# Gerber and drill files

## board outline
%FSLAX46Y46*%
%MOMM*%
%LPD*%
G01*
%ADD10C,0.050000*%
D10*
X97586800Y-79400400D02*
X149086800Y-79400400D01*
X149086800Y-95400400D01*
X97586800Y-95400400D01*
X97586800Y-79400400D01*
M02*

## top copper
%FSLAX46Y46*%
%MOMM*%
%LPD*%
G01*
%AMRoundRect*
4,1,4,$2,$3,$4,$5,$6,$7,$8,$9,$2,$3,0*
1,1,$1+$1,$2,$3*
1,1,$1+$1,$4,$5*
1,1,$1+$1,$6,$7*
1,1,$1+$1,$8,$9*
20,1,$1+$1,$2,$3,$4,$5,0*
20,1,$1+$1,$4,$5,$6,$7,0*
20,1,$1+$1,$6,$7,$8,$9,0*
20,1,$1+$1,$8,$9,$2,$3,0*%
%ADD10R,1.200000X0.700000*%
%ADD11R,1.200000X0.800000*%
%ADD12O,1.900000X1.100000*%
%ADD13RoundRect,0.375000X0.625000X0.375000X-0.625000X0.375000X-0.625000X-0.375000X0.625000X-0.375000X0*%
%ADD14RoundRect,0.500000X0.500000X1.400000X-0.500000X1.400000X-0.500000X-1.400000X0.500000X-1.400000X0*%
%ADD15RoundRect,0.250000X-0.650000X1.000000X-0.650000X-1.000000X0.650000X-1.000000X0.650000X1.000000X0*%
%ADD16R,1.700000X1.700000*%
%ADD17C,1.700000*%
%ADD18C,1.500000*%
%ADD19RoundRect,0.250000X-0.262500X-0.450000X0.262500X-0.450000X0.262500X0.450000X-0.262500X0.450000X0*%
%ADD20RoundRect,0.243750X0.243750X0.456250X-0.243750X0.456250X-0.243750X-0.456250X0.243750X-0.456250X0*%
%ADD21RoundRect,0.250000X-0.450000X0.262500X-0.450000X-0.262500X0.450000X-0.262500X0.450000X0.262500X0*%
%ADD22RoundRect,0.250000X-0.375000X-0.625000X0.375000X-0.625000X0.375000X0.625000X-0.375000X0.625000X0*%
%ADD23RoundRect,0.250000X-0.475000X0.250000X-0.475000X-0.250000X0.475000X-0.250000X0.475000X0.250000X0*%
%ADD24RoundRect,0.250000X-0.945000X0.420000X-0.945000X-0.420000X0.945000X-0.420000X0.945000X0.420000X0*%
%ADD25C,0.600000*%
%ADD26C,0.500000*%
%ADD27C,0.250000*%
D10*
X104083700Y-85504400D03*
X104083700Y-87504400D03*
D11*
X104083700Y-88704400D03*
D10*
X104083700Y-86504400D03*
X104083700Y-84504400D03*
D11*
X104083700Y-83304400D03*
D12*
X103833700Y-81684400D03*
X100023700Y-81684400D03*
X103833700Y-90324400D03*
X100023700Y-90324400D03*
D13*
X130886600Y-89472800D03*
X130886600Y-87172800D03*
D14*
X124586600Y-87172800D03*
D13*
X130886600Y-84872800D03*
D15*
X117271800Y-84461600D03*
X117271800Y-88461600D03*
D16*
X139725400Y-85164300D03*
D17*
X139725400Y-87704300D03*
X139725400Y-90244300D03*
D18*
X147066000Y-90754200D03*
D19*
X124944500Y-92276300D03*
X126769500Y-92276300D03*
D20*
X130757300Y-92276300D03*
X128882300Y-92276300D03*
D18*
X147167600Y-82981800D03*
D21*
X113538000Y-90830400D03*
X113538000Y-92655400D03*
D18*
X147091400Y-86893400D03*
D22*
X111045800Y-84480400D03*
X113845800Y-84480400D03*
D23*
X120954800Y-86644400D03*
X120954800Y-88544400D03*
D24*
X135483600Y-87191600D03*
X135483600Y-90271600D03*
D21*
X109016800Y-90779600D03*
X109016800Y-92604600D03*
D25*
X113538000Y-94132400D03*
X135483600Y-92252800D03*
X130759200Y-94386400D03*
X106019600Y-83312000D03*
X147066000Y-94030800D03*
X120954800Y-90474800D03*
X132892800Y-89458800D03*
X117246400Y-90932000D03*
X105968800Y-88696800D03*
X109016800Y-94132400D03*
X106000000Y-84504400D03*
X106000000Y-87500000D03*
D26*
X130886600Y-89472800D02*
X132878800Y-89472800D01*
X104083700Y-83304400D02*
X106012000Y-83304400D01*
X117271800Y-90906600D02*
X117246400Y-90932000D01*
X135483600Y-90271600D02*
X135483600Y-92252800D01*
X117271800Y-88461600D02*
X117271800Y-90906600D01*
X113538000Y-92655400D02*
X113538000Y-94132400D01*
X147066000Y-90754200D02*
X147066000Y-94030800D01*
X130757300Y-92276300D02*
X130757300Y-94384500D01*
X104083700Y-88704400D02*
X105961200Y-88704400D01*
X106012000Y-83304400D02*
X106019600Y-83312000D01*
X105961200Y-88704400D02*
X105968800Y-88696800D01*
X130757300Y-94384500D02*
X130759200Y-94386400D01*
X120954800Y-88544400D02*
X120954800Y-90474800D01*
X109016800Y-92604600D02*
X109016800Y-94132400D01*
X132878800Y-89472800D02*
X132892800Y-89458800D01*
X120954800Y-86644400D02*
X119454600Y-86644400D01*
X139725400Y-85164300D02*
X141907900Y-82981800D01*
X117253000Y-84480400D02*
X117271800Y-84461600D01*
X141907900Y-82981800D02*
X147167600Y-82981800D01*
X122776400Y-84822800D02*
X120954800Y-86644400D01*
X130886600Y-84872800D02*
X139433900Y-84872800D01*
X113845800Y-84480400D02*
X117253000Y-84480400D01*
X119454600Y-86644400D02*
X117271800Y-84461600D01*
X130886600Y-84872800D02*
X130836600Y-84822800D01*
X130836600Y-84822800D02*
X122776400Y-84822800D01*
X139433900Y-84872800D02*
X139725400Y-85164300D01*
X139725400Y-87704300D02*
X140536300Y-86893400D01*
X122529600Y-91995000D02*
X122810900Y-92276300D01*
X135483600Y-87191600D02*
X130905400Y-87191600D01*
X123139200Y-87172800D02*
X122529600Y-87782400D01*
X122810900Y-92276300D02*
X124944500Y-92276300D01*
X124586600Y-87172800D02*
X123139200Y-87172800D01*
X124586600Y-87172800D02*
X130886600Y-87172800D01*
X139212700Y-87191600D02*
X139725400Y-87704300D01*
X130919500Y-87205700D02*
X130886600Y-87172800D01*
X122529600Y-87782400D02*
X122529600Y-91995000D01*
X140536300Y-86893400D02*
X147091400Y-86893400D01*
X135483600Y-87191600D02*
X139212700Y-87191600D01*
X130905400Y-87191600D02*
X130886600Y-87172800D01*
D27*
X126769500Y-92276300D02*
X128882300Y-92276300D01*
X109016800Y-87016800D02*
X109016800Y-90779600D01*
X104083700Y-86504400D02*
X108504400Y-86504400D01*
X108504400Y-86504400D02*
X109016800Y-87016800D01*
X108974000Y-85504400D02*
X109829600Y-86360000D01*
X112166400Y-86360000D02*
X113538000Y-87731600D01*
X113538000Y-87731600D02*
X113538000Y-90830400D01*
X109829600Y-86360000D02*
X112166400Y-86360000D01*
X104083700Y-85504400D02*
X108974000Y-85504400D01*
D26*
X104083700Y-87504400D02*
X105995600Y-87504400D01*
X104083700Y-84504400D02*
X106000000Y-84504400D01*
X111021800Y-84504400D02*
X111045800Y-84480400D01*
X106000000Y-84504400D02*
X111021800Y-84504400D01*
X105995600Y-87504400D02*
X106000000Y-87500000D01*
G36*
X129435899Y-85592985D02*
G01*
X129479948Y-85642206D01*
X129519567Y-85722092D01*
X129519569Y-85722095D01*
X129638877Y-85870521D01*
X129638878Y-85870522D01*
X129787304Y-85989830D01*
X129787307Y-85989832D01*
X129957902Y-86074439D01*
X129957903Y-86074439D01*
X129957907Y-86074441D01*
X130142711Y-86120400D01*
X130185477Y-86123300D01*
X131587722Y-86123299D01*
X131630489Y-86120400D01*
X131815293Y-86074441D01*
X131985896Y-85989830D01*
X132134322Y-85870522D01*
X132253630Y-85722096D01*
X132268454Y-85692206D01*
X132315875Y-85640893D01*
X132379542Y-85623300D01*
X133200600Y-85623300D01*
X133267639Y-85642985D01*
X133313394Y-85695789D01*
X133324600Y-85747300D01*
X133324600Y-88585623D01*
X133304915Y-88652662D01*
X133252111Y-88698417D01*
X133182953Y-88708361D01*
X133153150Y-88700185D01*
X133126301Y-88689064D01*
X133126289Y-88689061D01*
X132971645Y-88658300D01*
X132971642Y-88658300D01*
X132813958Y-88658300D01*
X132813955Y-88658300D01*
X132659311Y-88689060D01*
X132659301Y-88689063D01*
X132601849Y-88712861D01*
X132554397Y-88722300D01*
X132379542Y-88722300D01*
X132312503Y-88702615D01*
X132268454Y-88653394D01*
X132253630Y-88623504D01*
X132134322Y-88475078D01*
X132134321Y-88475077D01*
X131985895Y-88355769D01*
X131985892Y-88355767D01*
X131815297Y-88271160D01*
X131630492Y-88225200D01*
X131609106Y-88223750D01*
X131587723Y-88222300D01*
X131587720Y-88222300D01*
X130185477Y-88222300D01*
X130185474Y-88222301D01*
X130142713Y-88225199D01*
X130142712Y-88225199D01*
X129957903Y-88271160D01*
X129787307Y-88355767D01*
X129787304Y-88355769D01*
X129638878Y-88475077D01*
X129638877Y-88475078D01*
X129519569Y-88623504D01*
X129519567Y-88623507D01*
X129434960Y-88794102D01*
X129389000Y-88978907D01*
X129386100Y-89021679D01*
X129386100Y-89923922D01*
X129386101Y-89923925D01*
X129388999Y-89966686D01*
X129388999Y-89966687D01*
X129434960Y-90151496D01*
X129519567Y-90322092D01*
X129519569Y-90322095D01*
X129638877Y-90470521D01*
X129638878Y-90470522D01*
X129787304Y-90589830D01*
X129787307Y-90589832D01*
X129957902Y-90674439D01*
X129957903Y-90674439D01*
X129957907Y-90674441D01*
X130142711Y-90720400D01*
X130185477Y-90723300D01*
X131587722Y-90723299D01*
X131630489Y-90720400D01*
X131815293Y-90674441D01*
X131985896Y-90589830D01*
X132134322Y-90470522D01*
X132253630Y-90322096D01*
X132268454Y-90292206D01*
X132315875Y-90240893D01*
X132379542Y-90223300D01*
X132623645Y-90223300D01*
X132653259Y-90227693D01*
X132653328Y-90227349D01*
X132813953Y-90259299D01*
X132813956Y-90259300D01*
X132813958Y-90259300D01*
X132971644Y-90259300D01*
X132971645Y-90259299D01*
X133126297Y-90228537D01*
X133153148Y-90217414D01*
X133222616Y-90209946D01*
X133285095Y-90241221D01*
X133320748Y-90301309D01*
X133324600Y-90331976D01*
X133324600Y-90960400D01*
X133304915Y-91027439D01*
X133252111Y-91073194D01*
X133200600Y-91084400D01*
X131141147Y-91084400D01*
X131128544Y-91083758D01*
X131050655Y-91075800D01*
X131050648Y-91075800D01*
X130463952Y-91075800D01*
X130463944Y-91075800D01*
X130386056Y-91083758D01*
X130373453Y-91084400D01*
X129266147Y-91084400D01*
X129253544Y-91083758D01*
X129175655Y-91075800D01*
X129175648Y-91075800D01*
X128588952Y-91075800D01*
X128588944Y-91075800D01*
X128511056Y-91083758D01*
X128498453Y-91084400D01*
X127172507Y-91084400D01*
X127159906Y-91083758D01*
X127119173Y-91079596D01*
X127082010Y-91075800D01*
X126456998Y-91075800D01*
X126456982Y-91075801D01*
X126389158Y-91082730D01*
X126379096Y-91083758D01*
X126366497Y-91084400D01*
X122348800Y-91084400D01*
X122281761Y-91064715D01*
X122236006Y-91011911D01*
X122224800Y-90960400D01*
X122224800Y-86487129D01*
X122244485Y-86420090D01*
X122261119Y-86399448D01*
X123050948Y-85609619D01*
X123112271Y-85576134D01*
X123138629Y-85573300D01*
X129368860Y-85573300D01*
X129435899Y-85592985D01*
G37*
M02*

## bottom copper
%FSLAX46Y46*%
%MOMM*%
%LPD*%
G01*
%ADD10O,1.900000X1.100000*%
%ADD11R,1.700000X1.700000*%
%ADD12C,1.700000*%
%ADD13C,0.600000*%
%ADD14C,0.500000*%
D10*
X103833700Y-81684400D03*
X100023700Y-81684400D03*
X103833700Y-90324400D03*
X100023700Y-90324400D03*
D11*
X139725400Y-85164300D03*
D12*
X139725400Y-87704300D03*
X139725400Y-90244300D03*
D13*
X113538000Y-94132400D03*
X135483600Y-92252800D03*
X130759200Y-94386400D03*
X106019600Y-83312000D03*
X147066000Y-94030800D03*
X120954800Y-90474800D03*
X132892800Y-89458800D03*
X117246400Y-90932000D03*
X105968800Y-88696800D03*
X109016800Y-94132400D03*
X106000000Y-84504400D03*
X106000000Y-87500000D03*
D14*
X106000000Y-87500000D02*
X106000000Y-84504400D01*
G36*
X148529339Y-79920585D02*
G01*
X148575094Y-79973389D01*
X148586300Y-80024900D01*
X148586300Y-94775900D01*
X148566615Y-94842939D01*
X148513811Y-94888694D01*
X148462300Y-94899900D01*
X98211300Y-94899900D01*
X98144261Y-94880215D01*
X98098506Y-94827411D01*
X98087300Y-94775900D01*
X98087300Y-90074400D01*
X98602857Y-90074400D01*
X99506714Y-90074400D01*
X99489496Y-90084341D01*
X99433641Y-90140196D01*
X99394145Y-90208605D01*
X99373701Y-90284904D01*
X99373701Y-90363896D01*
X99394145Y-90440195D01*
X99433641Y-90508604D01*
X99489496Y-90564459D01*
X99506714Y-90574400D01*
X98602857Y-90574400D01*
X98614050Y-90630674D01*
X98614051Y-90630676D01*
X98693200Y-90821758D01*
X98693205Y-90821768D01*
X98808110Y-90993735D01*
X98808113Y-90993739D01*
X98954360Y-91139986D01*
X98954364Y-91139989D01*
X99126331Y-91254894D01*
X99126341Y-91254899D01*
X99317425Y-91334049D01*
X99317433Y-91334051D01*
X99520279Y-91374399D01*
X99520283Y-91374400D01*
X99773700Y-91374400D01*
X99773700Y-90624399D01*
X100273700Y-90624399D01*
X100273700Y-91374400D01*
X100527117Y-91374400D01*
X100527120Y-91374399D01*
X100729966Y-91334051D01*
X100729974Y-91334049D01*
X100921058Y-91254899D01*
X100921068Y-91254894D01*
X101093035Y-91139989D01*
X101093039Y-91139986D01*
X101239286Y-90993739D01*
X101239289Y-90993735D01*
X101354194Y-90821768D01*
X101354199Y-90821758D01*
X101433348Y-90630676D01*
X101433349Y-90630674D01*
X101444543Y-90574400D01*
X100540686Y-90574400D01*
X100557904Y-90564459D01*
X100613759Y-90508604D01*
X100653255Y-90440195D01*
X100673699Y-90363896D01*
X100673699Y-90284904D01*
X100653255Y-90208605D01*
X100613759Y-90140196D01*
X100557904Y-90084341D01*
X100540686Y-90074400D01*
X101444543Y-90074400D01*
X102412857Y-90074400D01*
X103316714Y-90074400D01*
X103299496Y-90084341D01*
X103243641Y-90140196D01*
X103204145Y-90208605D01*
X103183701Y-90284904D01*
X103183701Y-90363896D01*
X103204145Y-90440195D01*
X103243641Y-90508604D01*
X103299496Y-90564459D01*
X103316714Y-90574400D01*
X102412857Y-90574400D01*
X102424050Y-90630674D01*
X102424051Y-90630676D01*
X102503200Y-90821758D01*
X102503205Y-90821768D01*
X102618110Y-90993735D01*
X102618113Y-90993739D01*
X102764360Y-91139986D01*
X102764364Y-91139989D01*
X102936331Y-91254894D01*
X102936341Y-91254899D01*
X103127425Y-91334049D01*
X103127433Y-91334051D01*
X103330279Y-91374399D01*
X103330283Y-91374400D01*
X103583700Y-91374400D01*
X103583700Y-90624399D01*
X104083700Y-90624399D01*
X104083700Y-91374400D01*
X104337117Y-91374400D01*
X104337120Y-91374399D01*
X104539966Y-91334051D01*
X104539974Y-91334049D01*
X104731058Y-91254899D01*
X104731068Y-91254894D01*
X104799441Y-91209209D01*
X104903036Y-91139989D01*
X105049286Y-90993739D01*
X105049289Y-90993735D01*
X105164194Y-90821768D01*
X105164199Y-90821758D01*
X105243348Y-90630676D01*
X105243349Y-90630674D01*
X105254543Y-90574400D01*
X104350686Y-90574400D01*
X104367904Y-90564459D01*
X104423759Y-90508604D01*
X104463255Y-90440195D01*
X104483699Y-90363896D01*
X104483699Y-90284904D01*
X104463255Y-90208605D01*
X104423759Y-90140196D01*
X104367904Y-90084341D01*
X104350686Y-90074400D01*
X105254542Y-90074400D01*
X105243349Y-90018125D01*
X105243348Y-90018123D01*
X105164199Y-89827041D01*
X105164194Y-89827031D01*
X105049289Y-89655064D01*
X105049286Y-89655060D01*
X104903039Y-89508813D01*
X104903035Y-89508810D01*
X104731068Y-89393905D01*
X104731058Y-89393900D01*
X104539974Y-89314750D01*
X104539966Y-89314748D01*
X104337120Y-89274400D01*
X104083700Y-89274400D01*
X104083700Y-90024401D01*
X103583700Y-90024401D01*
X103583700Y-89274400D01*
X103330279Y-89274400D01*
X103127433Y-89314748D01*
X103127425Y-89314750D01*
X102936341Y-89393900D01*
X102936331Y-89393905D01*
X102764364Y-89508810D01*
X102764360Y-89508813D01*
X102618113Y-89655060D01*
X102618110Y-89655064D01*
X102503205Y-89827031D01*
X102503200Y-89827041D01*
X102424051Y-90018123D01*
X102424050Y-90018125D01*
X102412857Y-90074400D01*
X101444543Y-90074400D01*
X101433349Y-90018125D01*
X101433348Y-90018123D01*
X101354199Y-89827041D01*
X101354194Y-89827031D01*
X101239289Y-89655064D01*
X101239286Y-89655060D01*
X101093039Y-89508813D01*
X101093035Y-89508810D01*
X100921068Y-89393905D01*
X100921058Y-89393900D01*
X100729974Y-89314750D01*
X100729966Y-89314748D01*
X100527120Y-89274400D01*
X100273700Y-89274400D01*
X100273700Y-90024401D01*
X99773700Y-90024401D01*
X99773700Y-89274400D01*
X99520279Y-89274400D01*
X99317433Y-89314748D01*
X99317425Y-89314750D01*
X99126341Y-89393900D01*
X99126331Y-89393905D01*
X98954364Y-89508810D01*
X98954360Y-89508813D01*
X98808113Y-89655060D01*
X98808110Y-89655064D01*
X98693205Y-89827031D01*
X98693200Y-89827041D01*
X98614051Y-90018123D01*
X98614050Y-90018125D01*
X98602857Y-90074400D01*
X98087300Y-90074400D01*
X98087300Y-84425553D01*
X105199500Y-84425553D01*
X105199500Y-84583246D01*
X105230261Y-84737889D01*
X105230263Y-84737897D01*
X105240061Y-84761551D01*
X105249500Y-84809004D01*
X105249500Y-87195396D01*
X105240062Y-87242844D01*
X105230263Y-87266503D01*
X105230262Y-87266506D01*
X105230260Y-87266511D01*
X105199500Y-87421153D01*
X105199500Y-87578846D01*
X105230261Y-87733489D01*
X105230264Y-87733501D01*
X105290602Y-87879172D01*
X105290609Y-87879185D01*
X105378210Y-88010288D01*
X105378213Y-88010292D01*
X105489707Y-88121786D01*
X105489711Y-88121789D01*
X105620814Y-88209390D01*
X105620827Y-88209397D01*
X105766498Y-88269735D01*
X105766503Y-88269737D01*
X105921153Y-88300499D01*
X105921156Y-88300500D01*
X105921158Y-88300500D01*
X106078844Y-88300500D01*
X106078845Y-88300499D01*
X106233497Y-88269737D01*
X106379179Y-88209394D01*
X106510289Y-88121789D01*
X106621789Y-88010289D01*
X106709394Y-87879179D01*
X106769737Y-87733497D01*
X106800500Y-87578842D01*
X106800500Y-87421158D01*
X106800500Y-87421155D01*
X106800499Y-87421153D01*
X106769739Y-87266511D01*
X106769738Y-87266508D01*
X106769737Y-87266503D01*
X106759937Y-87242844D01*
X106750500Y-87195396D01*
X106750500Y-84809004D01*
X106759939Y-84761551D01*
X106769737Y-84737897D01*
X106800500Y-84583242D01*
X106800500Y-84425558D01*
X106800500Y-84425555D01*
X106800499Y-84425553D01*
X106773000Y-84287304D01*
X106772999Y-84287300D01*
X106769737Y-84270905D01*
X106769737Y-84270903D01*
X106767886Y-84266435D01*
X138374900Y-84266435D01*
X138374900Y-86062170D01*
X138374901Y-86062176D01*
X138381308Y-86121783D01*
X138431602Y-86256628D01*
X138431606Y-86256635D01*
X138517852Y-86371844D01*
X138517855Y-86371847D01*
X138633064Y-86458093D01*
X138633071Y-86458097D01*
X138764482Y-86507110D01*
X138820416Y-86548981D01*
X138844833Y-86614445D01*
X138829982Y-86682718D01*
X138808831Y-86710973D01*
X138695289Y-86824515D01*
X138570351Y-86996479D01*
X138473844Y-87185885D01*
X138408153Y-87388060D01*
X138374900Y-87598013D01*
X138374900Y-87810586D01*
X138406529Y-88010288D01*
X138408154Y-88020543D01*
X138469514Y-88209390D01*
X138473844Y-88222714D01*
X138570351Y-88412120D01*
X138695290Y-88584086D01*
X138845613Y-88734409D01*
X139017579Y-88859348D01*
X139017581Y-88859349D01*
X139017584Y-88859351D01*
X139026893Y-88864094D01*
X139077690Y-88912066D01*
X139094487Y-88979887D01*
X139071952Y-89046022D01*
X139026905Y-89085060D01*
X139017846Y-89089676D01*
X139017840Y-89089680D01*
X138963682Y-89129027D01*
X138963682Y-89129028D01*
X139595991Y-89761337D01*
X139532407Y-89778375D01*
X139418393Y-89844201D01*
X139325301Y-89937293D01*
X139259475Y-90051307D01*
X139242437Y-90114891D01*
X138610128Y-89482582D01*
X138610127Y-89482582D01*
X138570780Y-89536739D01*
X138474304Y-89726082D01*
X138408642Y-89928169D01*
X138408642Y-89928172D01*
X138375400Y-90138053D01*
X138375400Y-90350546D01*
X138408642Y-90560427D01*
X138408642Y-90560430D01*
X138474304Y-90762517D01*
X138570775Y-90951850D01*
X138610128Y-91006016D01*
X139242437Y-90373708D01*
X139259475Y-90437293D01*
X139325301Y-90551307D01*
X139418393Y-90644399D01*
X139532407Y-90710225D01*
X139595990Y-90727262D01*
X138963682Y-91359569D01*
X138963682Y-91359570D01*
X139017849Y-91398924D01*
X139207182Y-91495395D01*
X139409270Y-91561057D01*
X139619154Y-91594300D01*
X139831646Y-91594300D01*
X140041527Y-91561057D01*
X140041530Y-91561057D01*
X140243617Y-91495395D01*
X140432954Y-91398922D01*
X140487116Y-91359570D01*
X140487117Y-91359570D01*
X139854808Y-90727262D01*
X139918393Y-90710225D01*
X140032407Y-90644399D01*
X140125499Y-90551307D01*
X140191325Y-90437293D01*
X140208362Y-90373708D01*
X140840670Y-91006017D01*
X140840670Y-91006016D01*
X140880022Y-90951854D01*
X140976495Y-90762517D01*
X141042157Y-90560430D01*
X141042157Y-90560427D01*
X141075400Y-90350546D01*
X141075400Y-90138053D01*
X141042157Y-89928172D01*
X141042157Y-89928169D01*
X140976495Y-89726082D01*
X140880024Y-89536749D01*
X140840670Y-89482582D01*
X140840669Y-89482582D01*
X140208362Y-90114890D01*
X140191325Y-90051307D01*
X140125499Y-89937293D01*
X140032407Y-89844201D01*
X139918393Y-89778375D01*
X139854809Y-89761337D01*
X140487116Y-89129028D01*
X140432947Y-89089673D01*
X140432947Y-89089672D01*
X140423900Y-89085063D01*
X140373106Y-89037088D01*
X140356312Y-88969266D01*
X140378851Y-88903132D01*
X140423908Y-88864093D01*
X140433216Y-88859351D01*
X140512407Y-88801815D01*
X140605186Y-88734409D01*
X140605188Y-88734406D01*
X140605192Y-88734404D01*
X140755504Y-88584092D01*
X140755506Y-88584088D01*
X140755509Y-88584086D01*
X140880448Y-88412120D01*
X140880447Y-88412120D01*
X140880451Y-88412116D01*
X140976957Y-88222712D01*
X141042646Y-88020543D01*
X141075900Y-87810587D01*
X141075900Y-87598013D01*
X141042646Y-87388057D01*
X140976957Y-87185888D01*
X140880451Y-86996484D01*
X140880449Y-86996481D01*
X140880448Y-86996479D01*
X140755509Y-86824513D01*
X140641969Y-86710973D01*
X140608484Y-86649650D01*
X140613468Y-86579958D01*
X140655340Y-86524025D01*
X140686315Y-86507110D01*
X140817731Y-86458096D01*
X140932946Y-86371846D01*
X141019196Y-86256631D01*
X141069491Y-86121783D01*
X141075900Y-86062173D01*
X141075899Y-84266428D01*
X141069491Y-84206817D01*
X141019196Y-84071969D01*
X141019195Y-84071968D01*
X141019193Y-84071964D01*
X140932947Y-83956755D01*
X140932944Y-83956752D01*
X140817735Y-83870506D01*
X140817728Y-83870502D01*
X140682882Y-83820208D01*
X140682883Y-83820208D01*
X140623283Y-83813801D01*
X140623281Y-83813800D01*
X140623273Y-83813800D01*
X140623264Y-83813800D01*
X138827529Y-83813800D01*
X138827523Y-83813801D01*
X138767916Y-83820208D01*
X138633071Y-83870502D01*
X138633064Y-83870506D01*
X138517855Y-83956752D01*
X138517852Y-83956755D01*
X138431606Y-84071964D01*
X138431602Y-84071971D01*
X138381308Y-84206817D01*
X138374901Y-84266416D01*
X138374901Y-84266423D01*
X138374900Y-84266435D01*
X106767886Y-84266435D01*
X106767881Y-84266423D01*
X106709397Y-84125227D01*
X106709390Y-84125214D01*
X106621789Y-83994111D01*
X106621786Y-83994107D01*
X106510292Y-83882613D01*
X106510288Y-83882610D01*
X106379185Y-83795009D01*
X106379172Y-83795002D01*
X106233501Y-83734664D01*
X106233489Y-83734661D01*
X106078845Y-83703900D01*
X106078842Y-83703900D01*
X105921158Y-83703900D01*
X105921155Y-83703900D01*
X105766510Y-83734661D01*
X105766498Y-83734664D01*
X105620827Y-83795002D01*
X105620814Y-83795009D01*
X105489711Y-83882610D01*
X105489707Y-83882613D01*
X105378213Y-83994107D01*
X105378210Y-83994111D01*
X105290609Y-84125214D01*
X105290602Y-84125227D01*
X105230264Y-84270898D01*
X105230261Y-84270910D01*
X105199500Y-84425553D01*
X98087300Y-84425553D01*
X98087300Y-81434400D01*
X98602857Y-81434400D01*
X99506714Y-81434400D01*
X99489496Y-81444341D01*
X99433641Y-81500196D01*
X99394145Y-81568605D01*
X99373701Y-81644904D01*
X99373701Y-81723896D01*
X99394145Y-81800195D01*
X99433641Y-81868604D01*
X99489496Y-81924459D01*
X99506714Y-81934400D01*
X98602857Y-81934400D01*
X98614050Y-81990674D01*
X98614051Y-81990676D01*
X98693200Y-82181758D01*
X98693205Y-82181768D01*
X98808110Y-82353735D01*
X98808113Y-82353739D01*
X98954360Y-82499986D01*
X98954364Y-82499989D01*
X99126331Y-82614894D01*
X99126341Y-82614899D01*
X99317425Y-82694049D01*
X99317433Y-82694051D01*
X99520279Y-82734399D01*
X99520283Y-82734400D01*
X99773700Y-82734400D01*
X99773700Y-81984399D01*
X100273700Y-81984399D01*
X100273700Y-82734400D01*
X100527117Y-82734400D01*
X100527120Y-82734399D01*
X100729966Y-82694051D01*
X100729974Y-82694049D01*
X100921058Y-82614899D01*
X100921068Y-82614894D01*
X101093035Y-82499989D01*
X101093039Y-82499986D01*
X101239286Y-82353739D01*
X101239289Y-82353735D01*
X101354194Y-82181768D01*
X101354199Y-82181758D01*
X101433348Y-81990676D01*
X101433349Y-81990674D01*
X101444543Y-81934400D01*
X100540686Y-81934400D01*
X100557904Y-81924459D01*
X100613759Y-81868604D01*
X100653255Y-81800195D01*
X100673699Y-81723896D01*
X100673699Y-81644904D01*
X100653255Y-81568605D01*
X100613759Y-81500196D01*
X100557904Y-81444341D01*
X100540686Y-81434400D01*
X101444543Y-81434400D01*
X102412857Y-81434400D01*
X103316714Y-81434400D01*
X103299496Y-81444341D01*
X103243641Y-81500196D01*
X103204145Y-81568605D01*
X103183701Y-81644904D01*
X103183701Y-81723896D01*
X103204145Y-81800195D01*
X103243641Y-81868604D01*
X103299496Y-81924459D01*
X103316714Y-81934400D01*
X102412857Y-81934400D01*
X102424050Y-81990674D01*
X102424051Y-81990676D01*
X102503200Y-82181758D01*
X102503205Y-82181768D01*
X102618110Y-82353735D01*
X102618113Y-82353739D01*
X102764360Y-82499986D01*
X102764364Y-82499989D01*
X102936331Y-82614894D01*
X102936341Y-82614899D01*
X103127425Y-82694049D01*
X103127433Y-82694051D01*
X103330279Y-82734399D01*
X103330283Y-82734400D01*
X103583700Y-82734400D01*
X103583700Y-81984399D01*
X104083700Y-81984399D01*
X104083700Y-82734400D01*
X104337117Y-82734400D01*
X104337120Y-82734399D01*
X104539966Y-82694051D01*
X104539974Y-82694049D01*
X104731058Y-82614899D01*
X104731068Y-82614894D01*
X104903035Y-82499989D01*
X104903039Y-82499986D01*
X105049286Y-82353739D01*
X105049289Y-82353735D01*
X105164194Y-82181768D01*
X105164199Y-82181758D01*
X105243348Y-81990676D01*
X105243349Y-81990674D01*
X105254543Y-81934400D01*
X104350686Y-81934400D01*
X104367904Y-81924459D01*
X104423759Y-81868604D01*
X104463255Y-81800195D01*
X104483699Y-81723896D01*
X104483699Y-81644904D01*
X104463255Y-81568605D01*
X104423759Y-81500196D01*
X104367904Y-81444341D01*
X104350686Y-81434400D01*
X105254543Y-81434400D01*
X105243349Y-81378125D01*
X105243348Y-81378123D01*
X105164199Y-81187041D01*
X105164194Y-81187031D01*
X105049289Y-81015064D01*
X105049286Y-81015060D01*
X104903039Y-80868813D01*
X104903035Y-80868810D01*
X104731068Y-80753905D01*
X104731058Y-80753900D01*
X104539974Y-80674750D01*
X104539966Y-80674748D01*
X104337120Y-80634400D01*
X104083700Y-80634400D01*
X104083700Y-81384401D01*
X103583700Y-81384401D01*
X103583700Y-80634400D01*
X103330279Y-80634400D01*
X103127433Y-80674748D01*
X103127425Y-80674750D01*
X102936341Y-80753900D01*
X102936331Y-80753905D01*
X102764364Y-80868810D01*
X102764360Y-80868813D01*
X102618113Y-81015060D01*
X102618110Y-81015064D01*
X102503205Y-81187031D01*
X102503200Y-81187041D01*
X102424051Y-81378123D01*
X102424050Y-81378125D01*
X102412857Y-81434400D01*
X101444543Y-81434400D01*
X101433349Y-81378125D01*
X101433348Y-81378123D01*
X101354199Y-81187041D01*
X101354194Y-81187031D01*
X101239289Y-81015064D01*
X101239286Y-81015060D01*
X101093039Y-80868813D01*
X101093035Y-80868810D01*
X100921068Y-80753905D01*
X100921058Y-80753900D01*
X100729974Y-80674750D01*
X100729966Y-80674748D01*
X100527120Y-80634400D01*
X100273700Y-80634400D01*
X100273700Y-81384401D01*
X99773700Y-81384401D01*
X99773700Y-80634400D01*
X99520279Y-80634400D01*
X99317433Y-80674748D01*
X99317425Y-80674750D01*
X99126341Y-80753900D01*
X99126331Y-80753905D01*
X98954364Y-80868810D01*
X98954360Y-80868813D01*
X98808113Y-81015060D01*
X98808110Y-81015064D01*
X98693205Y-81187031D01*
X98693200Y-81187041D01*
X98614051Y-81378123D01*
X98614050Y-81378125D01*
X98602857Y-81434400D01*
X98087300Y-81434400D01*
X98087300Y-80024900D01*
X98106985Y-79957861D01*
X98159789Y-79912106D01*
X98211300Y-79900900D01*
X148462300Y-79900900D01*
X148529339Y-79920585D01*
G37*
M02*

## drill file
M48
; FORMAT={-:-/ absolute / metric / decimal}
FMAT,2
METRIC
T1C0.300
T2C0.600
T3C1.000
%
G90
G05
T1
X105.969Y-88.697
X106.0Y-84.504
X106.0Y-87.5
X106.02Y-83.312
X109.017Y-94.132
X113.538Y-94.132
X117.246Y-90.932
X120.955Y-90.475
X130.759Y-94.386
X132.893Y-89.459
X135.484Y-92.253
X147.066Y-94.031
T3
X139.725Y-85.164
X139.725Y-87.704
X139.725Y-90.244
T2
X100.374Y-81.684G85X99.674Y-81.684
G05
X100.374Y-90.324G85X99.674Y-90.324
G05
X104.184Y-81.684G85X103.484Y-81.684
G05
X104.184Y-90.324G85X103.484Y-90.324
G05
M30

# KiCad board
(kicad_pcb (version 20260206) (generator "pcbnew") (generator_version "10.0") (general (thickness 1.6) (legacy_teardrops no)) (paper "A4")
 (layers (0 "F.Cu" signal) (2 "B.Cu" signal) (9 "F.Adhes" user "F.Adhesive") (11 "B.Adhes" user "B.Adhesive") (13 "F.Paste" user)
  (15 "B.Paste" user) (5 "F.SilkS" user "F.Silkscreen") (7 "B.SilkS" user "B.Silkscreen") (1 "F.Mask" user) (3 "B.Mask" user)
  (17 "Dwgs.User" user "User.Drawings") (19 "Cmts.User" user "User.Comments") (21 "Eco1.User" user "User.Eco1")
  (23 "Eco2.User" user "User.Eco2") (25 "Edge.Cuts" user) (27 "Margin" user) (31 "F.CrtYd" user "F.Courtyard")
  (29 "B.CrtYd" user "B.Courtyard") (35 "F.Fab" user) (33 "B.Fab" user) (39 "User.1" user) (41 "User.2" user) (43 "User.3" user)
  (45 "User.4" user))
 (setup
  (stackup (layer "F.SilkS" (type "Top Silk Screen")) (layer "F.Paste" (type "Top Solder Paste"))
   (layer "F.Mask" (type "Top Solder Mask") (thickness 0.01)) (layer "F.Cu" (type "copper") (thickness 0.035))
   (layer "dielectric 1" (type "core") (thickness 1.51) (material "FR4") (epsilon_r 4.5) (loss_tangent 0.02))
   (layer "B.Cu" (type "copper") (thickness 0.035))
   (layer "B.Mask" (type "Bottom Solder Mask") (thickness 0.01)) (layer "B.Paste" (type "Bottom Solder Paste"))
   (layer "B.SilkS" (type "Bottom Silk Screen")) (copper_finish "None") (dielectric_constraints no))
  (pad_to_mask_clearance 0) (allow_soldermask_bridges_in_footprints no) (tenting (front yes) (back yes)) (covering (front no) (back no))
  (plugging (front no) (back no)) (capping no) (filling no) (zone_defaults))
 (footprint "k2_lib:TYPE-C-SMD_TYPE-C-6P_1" (layer "F.Cu") (at 102.0537 86.0044 -90)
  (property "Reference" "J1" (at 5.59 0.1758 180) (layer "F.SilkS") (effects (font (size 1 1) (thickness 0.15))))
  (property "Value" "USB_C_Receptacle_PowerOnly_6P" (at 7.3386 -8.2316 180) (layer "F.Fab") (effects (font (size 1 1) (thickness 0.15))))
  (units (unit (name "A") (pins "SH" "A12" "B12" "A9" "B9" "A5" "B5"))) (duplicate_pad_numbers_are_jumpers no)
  (pad "A5" smd rect (at -0.5 -2.03 270) (size 0.7 1.2) (layers "F.Cu" "F.Mask" "F.Paste") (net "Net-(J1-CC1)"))
  (pad "A9" smd rect (at 1.5 -2.03 270) (size 0.7 1.2) (layers "F.Cu" "F.Mask" "F.Paste") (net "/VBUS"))
  (pad "A12" smd rect (at 2.7 -2.03 270) (size 0.8 1.2) (layers "F.Cu" "F.Mask" "F.Paste") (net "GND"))
  (pad "B5" smd rect (at 0.5 -2.03 270) (size 0.7 1.2) (layers "F.Cu" "F.Mask" "F.Paste") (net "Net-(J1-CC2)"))
  (pad "B9" smd rect (at -1.5 -2.03 270) (size 0.7 1.2) (layers "F.Cu" "F.Mask" "F.Paste") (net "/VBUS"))
  (pad "B12" smd rect (at -2.7 -2.03 270) (size 0.8 1.2) (layers "F.Cu" "F.Mask" "F.Paste") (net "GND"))
  (pad "SH" thru_hole oval (at -4.32 -1.78 270) (size 1.1 1.9) (drill oval 0.599998 1.299997) (layers "*.Cu" "*.Mask")
   (remove_unused_layers no) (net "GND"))
  (pad "SH" thru_hole oval (at -4.32 2.03 270) (size 1.1 1.9) (drill oval 0.599998 1.299997) (layers "*.Cu" "*.Mask")
   (remove_unused_layers no) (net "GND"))
  (pad "SH" thru_hole oval (at 4.32 -1.78 270) (size 1.1 1.9) (drill oval 0.599998 1.299997) (layers "*.Cu" "*.Mask")
   (remove_unused_layers no) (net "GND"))
  (pad "SH" thru_hole oval (at 4.32 2.03 270) (size 1.1 1.9) (drill oval 0.599998 1.299997) (layers "*.Cu" "*.Mask")
   (remove_unused_layers no) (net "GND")))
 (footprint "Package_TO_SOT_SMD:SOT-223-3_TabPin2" (layer "F.Cu") (at 127.7366 87.1728 180)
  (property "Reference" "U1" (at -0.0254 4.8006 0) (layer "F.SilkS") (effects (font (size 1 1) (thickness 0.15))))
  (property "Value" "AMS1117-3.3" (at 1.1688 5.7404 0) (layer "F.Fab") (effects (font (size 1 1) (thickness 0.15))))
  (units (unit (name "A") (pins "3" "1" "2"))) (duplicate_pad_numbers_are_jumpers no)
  (pad "1" smd roundrect (at -3.15 -2.3 180) (size 2 1.5) (layers "F.Cu" "F.Mask" "F.Paste") (roundrect_rratio 0.25) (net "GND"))
  (pad "2" smd roundrect (at -3.15 0 180) (size 2 1.5) (layers "F.Cu" "F.Mask" "F.Paste") (roundrect_rratio 0.25) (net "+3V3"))
  (pad "2" smd roundrect (at 3.15 0 180) (size 2 3.8) (layers "F.Cu" "F.Mask" "F.Paste") (roundrect_rratio 0.25) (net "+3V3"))
  (pad "3" smd roundrect (at -3.15 2.3 180) (size 2 1.5) (layers "F.Cu" "F.Mask" "F.Paste") (roundrect_rratio 0.25) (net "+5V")))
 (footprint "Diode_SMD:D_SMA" (layer "F.Cu") (at 117.2718 86.4616 -90)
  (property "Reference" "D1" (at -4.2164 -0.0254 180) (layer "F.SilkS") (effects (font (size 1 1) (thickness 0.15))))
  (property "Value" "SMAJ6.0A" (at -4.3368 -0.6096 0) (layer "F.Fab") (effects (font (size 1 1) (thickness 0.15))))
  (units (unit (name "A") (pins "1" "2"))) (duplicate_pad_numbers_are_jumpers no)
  (pad "1" smd roundrect (at -2 0 270) (size 2.5 1.8) (layers "F.Cu" "F.Mask" "F.Paste") (roundrect_rratio 0.1388888889) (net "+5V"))
  (pad "2" smd roundrect (at 2 0 270) (size 2.5 1.8) (layers "F.Cu" "F.Mask" "F.Paste") (roundrect_rratio 0.1388888889) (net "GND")))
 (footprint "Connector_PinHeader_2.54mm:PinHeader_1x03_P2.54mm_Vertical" (layer "F.Cu") (at 139.7254 85.1643)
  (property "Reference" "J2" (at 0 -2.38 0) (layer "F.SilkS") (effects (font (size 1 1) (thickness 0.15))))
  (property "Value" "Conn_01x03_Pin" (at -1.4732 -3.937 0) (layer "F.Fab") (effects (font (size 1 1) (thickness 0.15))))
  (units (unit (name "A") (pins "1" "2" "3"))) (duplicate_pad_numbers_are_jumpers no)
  (pad "1" thru_hole rect (at 0 0) (size 1.7 1.7) (drill 1) (layers "*.Cu" "*.Mask") (remove_unused_layers no) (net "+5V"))
  (pad "2" thru_hole circle (at 0 2.54) (size 1.7 1.7) (drill 1) (layers "*.Cu" "*.Mask") (remove_unused_layers no) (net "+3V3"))
  (pad "3" thru_hole circle (at 0 5.08) (size 1.7 1.7) (drill 1) (layers "*.Cu" "*.Mask") (remove_unused_layers no) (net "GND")))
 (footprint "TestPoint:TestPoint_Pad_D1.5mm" (layer "F.Cu") (at 147.066 90.7542 180)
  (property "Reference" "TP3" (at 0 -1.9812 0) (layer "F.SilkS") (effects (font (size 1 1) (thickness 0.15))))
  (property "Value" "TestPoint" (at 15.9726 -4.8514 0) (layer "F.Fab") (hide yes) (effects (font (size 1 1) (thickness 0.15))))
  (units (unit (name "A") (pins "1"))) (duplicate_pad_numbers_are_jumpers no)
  (pad "1" smd circle (at 0 0 180) (size 1.5 1.5) (layers "F.Cu" "F.Mask") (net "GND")))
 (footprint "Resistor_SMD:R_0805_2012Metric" (layer "F.Cu") (at 125.857 92.2763)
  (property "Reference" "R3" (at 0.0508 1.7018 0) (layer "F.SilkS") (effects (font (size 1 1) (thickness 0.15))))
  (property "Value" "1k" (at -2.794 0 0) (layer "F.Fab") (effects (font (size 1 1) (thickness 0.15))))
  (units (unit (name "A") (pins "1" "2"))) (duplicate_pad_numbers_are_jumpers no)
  (pad "1" smd roundrect (at -0.9125 0) (size 1.025 1.4) (layers "F.Cu" "F.Mask" "F.Paste") (roundrect_rratio 0.243902) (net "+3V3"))
  (pad "2" smd roundrect (at 0.9125 0) (size 1.025 1.4) (layers "F.Cu" "F.Mask" "F.Paste") (roundrect_rratio 0.243902) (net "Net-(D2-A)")))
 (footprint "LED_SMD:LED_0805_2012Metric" (layer "F.Cu") (at 129.8198 92.2763 180)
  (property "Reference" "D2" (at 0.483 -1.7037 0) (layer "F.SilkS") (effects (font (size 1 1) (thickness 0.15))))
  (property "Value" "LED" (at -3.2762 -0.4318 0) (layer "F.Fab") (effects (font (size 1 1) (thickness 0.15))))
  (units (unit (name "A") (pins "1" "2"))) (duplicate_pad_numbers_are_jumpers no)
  (pad "1" smd roundrect (at -0.9375 0 180) (size 0.975 1.4) (layers "F.Cu" "F.Mask" "F.Paste") (roundrect_rratio 0.25) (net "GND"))
  (pad "2" smd roundrect (at 0.9375 0 180) (size 0.975 1.4) (layers "F.Cu" "F.Mask" "F.Paste") (roundrect_rratio 0.25) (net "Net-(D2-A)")))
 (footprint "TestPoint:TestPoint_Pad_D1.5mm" (layer "F.Cu") (at 147.1676 82.9818)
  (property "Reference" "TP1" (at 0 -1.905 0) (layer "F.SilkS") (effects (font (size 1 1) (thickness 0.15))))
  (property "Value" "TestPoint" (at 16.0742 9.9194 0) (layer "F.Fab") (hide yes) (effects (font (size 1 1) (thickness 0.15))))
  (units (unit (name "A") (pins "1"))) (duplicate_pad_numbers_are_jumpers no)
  (pad "1" smd circle (at 0 0) (size 1.5 1.5) (layers "F.Cu" "F.Mask") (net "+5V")))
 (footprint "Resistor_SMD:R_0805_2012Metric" (layer "F.Cu") (at 113.538 91.7429 -90)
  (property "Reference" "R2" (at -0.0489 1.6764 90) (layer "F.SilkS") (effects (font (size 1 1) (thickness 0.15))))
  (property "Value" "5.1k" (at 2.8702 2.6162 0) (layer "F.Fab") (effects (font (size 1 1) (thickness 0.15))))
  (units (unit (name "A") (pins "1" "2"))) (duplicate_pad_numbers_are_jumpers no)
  (pad "1" smd roundrect (at -0.9125 0 270) (size 1.025 1.4) (layers "F.Cu" "F.Mask" "F.Paste") (roundrect_rratio 0.243902)
   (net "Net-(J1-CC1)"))
  (pad "2" smd roundrect (at 0.9125 0 270) (size 1.025 1.4) (layers "F.Cu" "F.Mask" "F.Paste") (roundrect_rratio 0.243902) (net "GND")))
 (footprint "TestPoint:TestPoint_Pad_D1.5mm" (layer "F.Cu") (at 147.0914 86.8934)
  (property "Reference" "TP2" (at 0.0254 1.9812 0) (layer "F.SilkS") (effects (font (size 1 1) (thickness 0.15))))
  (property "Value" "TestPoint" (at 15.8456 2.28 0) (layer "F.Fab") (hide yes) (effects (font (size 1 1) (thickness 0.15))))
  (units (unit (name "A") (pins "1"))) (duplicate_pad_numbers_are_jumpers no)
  (pad "1" smd circle (at 0 0) (size 1.5 1.5) (layers "F.Cu" "F.Mask") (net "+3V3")))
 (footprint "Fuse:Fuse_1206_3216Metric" (layer "F.Cu") (at 112.4458 84.4804)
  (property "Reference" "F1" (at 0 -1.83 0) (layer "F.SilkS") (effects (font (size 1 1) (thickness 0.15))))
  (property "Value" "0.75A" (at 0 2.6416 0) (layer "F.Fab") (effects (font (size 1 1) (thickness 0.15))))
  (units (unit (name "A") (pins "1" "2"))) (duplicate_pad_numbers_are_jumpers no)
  (pad "1" smd roundrect (at -1.4 0) (size 1.25 1.75) (layers "F.Cu" "F.Mask" "F.Paste") (roundrect_rratio 0.2) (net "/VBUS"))
  (pad "2" smd roundrect (at 1.4 0) (size 1.25 1.75) (layers "F.Cu" "F.Mask" "F.Paste") (roundrect_rratio 0.2) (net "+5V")))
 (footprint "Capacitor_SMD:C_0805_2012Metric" (layer "F.Cu") (at 120.9548 87.5944 -90)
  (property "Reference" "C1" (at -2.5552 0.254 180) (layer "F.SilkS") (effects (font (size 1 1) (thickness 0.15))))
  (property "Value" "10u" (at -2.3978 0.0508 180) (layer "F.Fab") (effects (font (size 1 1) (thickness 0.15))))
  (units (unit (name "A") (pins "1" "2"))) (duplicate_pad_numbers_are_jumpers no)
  (pad "1" smd roundrect (at -0.95 0 270) (size 1 1.45) (layers "F.Cu" "F.Mask" "F.Paste") (roundrect_rratio 0.25) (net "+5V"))
  (pad "2" smd roundrect (at 0.95 0 270) (size 1 1.45) (layers "F.Cu" "F.Mask" "F.Paste") (roundrect_rratio 0.25) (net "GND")))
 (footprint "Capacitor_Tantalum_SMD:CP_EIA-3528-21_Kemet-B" (layer "F.Cu") (at 135.4836 88.7316 -90)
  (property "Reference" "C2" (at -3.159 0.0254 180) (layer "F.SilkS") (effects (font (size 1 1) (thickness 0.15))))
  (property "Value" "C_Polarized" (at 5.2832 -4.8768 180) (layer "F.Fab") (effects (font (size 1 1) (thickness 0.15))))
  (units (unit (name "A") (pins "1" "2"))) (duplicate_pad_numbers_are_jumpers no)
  (pad "1" smd roundrect (at -1.54 0 270) (size 1.34 2.39) (layers "F.Cu" "F.Mask" "F.Paste") (roundrect_rratio 0.186567) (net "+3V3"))
  (pad "2" smd roundrect (at 1.54 0 270) (size 1.34 2.39) (layers "F.Cu" "F.Mask" "F.Paste") (roundrect_rratio 0.186567) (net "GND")))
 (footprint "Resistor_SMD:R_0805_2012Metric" (layer "F.Cu") (at 109.0168 91.6921 -90)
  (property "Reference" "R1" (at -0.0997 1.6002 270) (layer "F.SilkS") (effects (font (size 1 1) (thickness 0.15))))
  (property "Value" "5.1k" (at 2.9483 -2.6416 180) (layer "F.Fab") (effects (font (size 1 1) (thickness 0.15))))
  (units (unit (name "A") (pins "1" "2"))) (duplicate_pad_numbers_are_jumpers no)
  (pad "1" smd roundrect (at -0.9125 0 270) (size 1.025 1.4) (layers "F.Cu" "F.Mask" "F.Paste") (roundrect_rratio 0.243902)
   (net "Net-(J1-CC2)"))
  (pad "2" smd roundrect (at 0.9125 0 270) (size 1.025 1.4) (layers "F.Cu" "F.Mask" "F.Paste") (roundrect_rratio 0.243902) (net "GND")))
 (gr_rect (start 97.5868 79.4004) (end 149.0868 95.4004) (stroke (width 0.05) (type solid)) (fill no) (layer "Edge.Cuts"))
 (segment (start 130.8866 89.4728) (end 132.8788 89.4728) (width 0.5) (layer "F.Cu") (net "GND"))
 (segment (start 104.0837 83.3044) (end 106.012 83.3044) (width 0.5) (layer "F.Cu") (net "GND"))
 (segment (start 117.2718 90.9066) (end 117.2464 90.932) (width 0.5) (layer "F.Cu") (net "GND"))
 (segment (start 135.4836 90.2716) (end 135.4836 92.2528) (width 0.5) (layer "F.Cu") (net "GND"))
 (segment (start 117.2718 88.4616) (end 117.2718 90.9066) (width 0.5) (layer "F.Cu") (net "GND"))
 (segment (start 113.538 92.6554) (end 113.538 94.1324) (width 0.5) (layer "F.Cu") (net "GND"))
 (segment (start 147.066 90.7542) (end 147.066 94.0308) (width 0.5) (layer "F.Cu") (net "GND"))
 (segment (start 130.7573 92.2763) (end 130.7573 94.3845) (width 0.5) (layer "F.Cu") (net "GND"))
 (segment (start 104.0837 88.7044) (end 105.9612 88.7044) (width 0.5) (layer "F.Cu") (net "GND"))
 (segment (start 106.012 83.3044) (end 106.0196 83.312) (width 0.5) (layer "F.Cu") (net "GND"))
 (segment (start 105.9612 88.7044) (end 105.9688 88.6968) (width 0.5) (layer "F.Cu") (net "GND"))
 (segment (start 130.7573 94.3845) (end 130.7592 94.3864) (width 0.5) (layer "F.Cu") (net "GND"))
 (segment (start 120.9548 88.5444) (end 120.9548 90.4748) (width 0.5) (layer "F.Cu") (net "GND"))
 (segment (start 109.0168 92.6046) (end 109.0168 94.1324) (width 0.5) (layer "F.Cu") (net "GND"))
 (segment (start 132.8788 89.4728) (end 132.8928 89.4588) (width 0.5) (layer "F.Cu") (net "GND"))
 (via (at 113.538 94.1324) (size 0.6) (drill 0.3) (layers "F.Cu" "B.Cu") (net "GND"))
 (via (at 135.4836 92.2528) (size 0.6) (drill 0.3) (layers "F.Cu" "B.Cu") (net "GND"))
 (via (at 130.7592 94.3864) (size 0.6) (drill 0.3) (layers "F.Cu" "B.Cu") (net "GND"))
 (via (at 106.0196 83.312) (size 0.6) (drill 0.3) (layers "F.Cu" "B.Cu") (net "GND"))
 (via (at 147.066 94.0308) (size 0.6) (drill 0.3) (layers "F.Cu" "B.Cu") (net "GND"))
 (via (at 120.9548 90.4748) (size 0.6) (drill 0.3) (layers "F.Cu" "B.Cu") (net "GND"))
 (via (at 132.8928 89.4588) (size 0.6) (drill 0.3) (layers "F.Cu" "B.Cu") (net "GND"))
 (via (at 117.2464 90.932) (size 0.6) (drill 0.3) (layers "F.Cu" "B.Cu") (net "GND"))
 (via (at 105.9688 88.6968) (size 0.6) (drill 0.3) (layers "F.Cu" "B.Cu") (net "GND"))
 (via (at 109.0168 94.1324) (size 0.6) (drill 0.3) (layers "F.Cu" "B.Cu") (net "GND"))
 (segment (start 120.9548 86.6444) (end 119.4546 86.6444) (width 0.5) (layer "F.Cu") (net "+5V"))
 (segment (start 139.7254 85.1643) (end 141.9079 82.9818) (width 0.5) (layer "F.Cu") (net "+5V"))
 (segment (start 117.253 84.4804) (end 117.2718 84.4616) (width 0.5) (layer "F.Cu") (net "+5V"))
 (segment (start 141.9079 82.9818) (end 147.1676 82.9818) (width 0.5) (layer "F.Cu") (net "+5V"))
 (segment (start 122.7764 84.8228) (end 120.9548 86.6444) (width 0.5) (layer "F.Cu") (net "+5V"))
 (segment (start 130.8866 84.8728) (end 139.4339 84.8728) (width 0.5) (layer "F.Cu") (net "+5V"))
 (segment (start 113.8458 84.4804) (end 117.253 84.4804) (width 0.5) (layer "F.Cu") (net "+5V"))
 (segment (start 119.4546 86.6444) (end 117.2718 84.4616) (width 0.5) (layer "F.Cu") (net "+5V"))
 (segment (start 130.8866 84.8728) (end 130.8366 84.8228) (width 0.5) (layer "F.Cu") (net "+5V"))
 (segment (start 130.8366 84.8228) (end 122.7764 84.8228) (width 0.5) (layer "F.Cu") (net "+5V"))
 (segment (start 139.4339 84.8728) (end 139.7254 85.1643) (width 0.5) (layer "F.Cu") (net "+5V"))
 (segment (start 139.7254 87.7043) (end 140.5363 86.8934) (width 0.5) (layer "F.Cu") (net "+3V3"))
 (segment (start 122.5296 91.995) (end 122.8109 92.2763) (width 0.5) (layer "F.Cu") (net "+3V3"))
 (segment (start 135.4836 87.1916) (end 130.9054 87.1916) (width 0.5) (layer "F.Cu") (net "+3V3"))
 (segment (start 123.1392 87.1728) (end 122.5296 87.7824) (width 0.5) (layer "F.Cu") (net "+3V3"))
 (segment (start 122.8109 92.2763) (end 124.9445 92.2763) (width 0.5) (layer "F.Cu") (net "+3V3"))
 (segment (start 124.5866 87.1728) (end 123.1392 87.1728) (width 0.5) (layer "F.Cu") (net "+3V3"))
 (segment (start 124.5866 87.1728) (end 130.8866 87.1728) (width 0.5) (layer "F.Cu") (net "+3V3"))
 (segment (start 139.2127 87.1916) (end 139.7254 87.7043) (width 0.5) (layer "F.Cu") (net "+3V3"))
 (segment (start 130.9195 87.2057) (end 130.8866 87.1728) (width 0.5) (layer "F.Cu") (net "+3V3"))
 (segment (start 122.5296 87.7824) (end 122.5296 91.995) (width 0.5) (layer "F.Cu") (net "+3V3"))
 (segment (start 140.5363 86.8934) (end 147.0914 86.8934) (width 0.5) (layer "F.Cu") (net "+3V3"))
 (segment (start 135.4836 87.1916) (end 139.2127 87.1916) (width 0.5) (layer "F.Cu") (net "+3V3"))
 (segment (start 130.9054 87.1916) (end 130.8866 87.1728) (width 0.5) (layer "F.Cu") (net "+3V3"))
 (segment (start 126.7695 92.2763) (end 128.8823 92.2763) (width 0.25) (layer "F.Cu") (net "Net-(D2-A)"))
 (segment (start 109.0168 87.0168) (end 109.0168 90.7796) (width 0.25) (layer "F.Cu") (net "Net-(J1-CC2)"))
 (segment (start 104.0837 86.5044) (end 108.5044 86.5044) (width 0.25) (layer "F.Cu") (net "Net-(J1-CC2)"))
 (segment (start 108.5044 86.5044) (end 109.0168 87.0168) (width 0.25) (layer "F.Cu") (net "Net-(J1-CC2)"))
 (segment (start 108.974 85.5044) (end 109.8296 86.36) (width 0.25) (layer "F.Cu") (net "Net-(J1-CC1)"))
 (segment (start 112.1664 86.36) (end 113.538 87.7316) (width 0.25) (layer "F.Cu") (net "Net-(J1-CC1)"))
 (segment (start 113.538 87.7316) (end 113.538 90.8304) (width 0.25) (layer "F.Cu") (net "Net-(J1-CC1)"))
 (segment (start 109.8296 86.36) (end 112.1664 86.36) (width 0.25) (layer "F.Cu") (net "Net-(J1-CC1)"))
 (segment (start 104.0837 85.5044) (end 108.974 85.5044) (width 0.25) (layer "F.Cu") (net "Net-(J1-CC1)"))
 (segment (start 104.0837 87.5044) (end 105.9956 87.5044) (width 0.5) (layer "F.Cu") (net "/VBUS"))
 (segment (start 104.0837 84.5044) (end 106 84.5044) (width 0.5) (layer "F.Cu") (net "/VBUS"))
 (segment (start 111.0218 84.5044) (end 111.0458 84.4804) (width 0.5) (layer "F.Cu") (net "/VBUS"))
 (segment (start 106 84.5044) (end 111.0218 84.5044) (width 0.5) (layer "F.Cu") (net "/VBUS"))
 (segment (start 105.9956 87.5044) (end 106 87.5) (width 0.5) (layer "F.Cu") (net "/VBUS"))
 (via (at 106 84.5044) (size 0.6) (drill 0.3) (layers "F.Cu" "B.Cu") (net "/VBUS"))
 (via (at 106 87.5) (size 0.6) (drill 0.3) (layers "F.Cu" "B.Cu") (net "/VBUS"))
 (segment (start 106 87.5) (end 106 84.5044) (width 0.5) (layer "B.Cu") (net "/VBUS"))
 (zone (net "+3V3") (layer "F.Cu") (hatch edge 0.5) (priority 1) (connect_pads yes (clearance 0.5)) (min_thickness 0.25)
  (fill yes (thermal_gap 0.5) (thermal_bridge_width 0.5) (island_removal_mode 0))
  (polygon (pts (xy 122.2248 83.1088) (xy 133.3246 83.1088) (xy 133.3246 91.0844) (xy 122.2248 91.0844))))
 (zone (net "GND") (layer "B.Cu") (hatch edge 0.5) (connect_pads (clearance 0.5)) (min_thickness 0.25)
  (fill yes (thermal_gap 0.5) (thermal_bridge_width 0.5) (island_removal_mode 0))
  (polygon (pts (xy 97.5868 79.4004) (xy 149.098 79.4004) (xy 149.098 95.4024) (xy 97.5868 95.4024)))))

